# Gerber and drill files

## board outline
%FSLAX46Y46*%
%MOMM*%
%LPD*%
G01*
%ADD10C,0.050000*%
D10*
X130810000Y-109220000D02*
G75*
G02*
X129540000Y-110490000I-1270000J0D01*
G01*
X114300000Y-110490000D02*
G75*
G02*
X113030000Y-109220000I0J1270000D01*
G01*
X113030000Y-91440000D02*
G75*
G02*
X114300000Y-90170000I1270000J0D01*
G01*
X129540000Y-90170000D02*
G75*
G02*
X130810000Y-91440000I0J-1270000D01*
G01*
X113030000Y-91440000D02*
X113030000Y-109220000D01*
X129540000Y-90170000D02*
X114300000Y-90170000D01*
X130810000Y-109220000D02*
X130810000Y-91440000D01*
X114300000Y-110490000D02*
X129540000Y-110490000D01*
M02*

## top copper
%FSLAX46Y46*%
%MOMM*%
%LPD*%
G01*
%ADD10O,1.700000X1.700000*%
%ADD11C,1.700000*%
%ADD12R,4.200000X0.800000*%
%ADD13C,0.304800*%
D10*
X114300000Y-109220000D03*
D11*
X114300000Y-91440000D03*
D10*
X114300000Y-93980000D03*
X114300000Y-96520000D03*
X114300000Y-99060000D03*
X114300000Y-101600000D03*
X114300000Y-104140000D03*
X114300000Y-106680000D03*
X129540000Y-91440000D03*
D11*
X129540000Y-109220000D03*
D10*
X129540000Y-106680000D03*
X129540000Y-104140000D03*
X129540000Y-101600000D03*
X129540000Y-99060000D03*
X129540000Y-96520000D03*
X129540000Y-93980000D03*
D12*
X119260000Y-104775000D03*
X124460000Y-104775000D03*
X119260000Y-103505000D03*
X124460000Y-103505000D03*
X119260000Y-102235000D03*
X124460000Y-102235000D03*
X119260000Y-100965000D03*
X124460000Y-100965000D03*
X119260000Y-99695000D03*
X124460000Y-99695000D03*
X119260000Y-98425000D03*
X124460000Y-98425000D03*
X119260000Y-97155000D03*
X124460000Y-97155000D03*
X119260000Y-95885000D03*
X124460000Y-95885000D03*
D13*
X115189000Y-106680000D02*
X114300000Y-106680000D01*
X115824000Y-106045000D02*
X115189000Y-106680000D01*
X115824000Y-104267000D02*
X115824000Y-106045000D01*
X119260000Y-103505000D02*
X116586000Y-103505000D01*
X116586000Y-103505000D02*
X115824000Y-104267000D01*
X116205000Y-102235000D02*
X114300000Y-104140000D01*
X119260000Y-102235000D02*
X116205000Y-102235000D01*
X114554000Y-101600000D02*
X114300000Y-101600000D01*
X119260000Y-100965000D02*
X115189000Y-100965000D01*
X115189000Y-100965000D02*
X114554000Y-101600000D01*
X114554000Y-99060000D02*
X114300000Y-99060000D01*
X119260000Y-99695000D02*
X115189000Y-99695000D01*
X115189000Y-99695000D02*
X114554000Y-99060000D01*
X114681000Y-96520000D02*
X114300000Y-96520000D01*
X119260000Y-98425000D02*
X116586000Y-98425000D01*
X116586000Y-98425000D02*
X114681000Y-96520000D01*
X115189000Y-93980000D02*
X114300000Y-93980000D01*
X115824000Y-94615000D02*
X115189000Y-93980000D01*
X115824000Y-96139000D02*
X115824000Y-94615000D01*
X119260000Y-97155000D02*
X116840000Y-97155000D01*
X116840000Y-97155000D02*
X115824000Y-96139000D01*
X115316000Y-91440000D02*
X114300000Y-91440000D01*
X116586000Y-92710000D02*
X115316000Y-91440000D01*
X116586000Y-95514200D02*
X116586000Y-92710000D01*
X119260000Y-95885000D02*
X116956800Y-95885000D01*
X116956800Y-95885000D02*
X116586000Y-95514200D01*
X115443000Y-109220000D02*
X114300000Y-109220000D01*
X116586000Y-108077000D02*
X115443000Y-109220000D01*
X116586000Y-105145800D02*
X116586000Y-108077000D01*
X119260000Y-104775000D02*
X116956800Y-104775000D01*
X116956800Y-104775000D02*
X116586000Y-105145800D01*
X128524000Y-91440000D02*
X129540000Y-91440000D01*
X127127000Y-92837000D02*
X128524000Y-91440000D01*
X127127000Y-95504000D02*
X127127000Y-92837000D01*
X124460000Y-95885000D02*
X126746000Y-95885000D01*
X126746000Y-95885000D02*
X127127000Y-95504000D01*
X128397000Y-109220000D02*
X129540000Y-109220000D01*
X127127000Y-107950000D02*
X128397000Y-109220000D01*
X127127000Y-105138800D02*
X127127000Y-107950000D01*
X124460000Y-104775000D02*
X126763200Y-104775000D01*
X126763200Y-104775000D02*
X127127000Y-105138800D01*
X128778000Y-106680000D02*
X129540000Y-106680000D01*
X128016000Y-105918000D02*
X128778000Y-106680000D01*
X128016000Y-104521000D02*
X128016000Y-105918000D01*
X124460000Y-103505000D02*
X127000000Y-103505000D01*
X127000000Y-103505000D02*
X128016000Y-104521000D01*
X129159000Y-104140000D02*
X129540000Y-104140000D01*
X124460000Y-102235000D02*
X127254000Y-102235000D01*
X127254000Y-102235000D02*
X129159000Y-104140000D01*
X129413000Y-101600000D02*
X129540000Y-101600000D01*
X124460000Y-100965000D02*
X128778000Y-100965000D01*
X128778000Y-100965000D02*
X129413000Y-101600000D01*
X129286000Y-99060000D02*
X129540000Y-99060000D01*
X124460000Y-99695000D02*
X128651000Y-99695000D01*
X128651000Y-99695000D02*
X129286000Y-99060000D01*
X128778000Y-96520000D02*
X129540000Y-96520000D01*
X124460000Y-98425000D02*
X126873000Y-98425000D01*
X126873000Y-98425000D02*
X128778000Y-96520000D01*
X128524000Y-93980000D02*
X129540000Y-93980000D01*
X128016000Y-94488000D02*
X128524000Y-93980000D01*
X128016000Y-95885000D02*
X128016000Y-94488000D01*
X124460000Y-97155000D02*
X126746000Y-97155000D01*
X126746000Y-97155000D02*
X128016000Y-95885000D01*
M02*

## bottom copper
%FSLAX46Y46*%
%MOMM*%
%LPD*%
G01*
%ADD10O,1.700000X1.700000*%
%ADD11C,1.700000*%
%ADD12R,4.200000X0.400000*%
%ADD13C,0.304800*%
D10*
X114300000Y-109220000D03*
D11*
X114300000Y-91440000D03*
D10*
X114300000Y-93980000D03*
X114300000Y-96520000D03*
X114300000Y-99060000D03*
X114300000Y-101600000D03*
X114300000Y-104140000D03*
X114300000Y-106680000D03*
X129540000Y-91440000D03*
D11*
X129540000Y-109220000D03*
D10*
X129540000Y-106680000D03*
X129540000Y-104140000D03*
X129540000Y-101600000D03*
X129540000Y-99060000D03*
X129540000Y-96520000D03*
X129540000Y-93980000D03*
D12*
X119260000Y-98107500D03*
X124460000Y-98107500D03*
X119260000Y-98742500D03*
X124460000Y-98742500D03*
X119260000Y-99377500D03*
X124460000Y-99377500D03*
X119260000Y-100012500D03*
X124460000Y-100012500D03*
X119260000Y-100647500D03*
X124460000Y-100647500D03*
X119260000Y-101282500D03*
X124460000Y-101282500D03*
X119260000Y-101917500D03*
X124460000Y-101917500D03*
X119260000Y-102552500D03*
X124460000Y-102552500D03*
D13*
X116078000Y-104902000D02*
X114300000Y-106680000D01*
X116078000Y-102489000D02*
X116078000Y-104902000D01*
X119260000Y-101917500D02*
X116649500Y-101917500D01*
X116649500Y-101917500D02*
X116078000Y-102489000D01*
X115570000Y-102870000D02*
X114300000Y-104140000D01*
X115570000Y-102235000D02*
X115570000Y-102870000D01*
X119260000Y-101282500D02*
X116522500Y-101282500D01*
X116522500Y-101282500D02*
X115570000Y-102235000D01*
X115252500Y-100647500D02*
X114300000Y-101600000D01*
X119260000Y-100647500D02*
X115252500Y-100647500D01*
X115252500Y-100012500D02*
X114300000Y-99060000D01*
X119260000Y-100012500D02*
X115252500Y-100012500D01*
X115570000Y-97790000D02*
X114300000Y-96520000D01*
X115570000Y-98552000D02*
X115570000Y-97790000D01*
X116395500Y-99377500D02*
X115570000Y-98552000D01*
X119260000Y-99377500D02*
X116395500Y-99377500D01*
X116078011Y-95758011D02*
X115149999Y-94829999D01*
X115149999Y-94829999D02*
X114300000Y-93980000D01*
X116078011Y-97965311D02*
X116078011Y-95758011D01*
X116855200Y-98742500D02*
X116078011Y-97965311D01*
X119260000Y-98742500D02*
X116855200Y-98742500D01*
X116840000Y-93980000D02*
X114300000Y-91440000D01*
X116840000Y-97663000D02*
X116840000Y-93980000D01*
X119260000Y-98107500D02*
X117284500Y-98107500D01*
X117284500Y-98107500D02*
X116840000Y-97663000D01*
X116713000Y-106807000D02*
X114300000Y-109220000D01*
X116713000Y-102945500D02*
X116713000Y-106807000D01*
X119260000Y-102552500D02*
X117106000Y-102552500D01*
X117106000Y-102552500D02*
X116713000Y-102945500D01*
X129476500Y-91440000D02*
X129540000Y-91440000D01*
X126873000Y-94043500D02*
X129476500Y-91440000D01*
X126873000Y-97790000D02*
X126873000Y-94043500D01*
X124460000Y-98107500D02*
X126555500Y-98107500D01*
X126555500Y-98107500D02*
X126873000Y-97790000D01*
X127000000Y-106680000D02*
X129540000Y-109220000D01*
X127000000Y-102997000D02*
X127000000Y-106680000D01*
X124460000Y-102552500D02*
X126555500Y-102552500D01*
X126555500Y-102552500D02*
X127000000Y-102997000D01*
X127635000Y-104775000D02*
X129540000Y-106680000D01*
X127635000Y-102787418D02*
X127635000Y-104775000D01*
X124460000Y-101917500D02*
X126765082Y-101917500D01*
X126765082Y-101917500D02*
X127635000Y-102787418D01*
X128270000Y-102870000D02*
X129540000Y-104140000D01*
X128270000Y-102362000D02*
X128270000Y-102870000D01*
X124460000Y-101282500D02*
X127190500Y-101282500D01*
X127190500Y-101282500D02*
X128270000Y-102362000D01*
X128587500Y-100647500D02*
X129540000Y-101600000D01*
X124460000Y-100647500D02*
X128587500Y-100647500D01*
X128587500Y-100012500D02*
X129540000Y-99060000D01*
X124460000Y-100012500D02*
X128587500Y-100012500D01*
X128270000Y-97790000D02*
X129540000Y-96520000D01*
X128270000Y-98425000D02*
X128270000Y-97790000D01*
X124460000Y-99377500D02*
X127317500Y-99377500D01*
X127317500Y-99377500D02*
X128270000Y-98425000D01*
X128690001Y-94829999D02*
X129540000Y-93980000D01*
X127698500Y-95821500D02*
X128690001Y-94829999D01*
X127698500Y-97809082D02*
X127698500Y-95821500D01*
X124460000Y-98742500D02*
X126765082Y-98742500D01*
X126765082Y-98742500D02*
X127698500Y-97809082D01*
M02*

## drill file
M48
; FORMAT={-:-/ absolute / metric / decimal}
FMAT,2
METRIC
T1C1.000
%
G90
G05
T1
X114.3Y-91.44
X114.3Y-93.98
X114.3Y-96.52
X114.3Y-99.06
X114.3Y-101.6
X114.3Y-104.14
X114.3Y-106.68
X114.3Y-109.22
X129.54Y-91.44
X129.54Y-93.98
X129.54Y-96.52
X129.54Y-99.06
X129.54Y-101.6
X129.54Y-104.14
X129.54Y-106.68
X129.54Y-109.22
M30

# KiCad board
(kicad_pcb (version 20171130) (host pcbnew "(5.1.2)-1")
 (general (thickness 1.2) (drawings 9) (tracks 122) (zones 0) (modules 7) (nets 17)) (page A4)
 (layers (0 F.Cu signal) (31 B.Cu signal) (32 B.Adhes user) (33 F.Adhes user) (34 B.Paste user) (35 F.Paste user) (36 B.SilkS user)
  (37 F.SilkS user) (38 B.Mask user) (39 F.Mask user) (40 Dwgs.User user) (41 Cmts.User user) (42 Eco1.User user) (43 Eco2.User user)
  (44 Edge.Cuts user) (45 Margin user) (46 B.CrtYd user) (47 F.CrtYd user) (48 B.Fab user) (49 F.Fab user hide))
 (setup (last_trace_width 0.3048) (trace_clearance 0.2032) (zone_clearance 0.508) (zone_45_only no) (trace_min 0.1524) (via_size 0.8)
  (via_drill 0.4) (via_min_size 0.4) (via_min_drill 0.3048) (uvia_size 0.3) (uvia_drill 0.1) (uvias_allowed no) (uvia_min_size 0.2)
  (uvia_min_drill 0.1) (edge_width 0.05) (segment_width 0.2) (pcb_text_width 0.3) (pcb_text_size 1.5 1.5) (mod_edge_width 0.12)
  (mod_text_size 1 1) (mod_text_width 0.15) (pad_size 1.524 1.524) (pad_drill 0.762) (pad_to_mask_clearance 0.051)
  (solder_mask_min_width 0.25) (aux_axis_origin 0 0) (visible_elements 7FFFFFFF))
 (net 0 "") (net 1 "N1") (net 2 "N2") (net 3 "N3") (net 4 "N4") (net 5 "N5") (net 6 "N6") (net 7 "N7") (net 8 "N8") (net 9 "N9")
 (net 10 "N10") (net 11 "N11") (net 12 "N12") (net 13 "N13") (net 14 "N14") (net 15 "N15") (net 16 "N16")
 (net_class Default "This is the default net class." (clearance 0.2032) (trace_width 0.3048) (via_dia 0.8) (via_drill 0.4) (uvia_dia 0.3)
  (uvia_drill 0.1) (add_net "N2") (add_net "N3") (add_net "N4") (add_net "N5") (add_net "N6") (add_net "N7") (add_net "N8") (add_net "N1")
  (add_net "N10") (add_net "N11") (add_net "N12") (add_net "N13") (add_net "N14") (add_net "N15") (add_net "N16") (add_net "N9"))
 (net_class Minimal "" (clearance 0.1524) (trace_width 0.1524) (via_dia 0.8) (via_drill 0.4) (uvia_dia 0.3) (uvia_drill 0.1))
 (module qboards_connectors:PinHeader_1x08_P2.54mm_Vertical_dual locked (layer F.Cu) (at 114.3 91.44)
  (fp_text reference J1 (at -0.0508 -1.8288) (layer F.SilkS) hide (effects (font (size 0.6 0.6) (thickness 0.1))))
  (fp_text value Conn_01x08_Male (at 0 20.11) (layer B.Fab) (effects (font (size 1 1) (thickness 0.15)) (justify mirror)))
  (pad 8 thru_hole oval (at 0 17.78) (size 1.7 1.7) (drill 1) (layers *.Cu *.Mask) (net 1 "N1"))
  (pad 1 thru_hole circle (at 0 0) (size 1.7 1.7) (drill 1) (layers *.Cu *.Mask) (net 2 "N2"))
  (pad 2 thru_hole oval (at 0 2.54) (size 1.7 1.7) (drill 1) (layers *.Cu *.Mask) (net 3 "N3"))
  (pad 3 thru_hole oval (at 0 5.08) (size 1.7 1.7) (drill 1) (layers *.Cu *.Mask) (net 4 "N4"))
  (pad 4 thru_hole oval (at 0 7.62) (size 1.7 1.7) (drill 1) (layers *.Cu *.Mask) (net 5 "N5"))
  (pad 5 thru_hole oval (at 0 10.16) (size 1.7 1.7) (drill 1) (layers *.Cu *.Mask) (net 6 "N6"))
  (pad 6 thru_hole oval (at 0 12.7) (size 1.7 1.7) (drill 1) (layers *.Cu *.Mask) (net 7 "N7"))
  (pad 7 thru_hole oval (at 0 15.24) (size 1.7 1.7) (drill 1) (layers *.Cu *.Mask) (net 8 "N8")))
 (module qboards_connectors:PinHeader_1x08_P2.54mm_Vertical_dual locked (layer F.Cu) (at 129.54 109.22 180)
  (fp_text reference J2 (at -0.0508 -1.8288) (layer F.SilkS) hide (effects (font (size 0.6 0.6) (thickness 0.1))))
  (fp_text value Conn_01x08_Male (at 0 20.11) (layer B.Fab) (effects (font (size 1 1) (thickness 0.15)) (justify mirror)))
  (pad 8 thru_hole oval (at 0 17.78 180) (size 1.7 1.7) (drill 1) (layers *.Cu *.Mask) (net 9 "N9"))
  (pad 1 thru_hole circle (at 0 0 180) (size 1.7 1.7) (drill 1) (layers *.Cu *.Mask) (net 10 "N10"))
  (pad 2 thru_hole oval (at 0 2.54 180) (size 1.7 1.7) (drill 1) (layers *.Cu *.Mask) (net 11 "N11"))
  (pad 3 thru_hole oval (at 0 5.08 180) (size 1.7 1.7) (drill 1) (layers *.Cu *.Mask) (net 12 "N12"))
  (pad 4 thru_hole oval (at 0 7.62 180) (size 1.7 1.7) (drill 1) (layers *.Cu *.Mask) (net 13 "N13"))
  (pad 5 thru_hole oval (at 0 10.16 180) (size 1.7 1.7) (drill 1) (layers *.Cu *.Mask) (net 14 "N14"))
  (pad 6 thru_hole oval (at 0 12.7 180) (size 1.7 1.7) (drill 1) (layers *.Cu *.Mask) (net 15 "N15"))
  (pad 7 thru_hole oval (at 0 15.24 180) (size 1.7 1.7) (drill 1) (layers *.Cu *.Mask) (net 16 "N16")))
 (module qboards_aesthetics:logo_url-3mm (layer F.Cu) (at 117.602 107.823)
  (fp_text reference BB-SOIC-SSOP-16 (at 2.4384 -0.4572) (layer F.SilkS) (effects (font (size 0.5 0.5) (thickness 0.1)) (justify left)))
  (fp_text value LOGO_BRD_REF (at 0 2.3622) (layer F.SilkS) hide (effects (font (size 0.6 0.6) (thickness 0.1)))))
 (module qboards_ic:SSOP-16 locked (layer B.Cu) (at 121.86 100.33 90)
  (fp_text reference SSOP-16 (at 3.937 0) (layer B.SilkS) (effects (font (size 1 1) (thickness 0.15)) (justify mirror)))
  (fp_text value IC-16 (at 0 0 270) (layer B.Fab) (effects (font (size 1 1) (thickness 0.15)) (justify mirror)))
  (pad 8 smd rect (at 2.2225 -2.6 90) (size 0.4 4.2) (layers B.Cu B.Paste B.Mask) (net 2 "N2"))
  (pad 9 smd rect (at 2.2225 2.6 90) (size 0.4 4.2) (layers B.Cu B.Paste B.Mask) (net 9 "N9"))
  (pad 7 smd rect (at 1.5875 -2.6 90) (size 0.4 4.2) (layers B.Cu B.Paste B.Mask) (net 3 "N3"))
  (pad 10 smd rect (at 1.5875 2.6 90) (size 0.4 4.2) (layers B.Cu B.Paste B.Mask) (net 16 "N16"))
  (pad 6 smd rect (at 0.9525 -2.6 90) (size 0.4 4.2) (layers B.Cu B.Paste B.Mask) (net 4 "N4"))
  (pad 11 smd rect (at 0.9525 2.6 90) (size 0.4 4.2) (layers B.Cu B.Paste B.Mask) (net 15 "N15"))
  (pad 5 smd rect (at 0.3175 -2.6 90) (size 0.4 4.2) (layers B.Cu B.Paste B.Mask) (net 5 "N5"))
  (pad 12 smd rect (at 0.3175 2.6 90) (size 0.4 4.2) (layers B.Cu B.Paste B.Mask) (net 14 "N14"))
  (pad 4 smd rect (at -0.3175 -2.6 90) (size 0.4 4.2) (layers B.Cu B.Paste B.Mask) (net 6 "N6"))
  (pad 13 smd rect (at -0.3175 2.6 90) (size 0.4 4.2) (layers B.Cu B.Paste B.Mask) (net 13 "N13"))
  (pad 3 smd rect (at -0.9525 -2.6 90) (size 0.4 4.2) (layers B.Cu B.Paste B.Mask) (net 7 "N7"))
  (pad 14 smd rect (at -0.9525 2.6 90) (size 0.4 4.2) (layers B.Cu B.Paste B.Mask) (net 12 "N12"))
  (pad 2 smd rect (at -1.5875 -2.6 90) (size 0.4 4.2) (layers B.Cu B.Paste B.Mask) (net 8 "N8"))
  (pad 15 smd rect (at -1.5875 2.6 90) (size 0.4 4.2) (layers B.Cu B.Paste B.Mask) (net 11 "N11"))
  (pad 1 smd rect (at -2.2225 -2.6 90) (size 0.4 4.2) (layers B.Cu B.Paste B.Mask) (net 1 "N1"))
  (pad 16 smd rect (at -2.2225 2.6 90) (size 0.4 4.2) (layers B.Cu B.Paste B.Mask) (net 10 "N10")))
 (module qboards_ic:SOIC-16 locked (layer F.Cu) (at 121.86 100.33 270)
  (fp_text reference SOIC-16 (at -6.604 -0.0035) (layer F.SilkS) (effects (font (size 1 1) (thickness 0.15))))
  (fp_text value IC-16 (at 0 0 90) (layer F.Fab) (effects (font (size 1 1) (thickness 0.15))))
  (pad 8 smd rect (at 4.445 2.6 270) (size 0.8 4.2) (layers F.Cu F.Paste F.Mask) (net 1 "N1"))
  (pad 9 smd rect (at 4.445 -2.6 270) (size 0.8 4.2) (layers F.Cu F.Paste F.Mask) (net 10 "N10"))
  (pad 7 smd rect (at 3.175 2.6 270) (size 0.8 4.2) (layers F.Cu F.Paste F.Mask) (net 8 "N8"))
  (pad 10 smd rect (at 3.175 -2.6 270) (size 0.8 4.2) (layers F.Cu F.Paste F.Mask) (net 11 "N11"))
  (pad 6 smd rect (at 1.905 2.6 270) (size 0.8 4.2) (layers F.Cu F.Paste F.Mask) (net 7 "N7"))
  (pad 11 smd rect (at 1.905 -2.6 270) (size 0.8 4.2) (layers F.Cu F.Paste F.Mask) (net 12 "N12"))
  (pad 5 smd rect (at 0.635 2.6 270) (size 0.8 4.2) (layers F.Cu F.Paste F.Mask) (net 6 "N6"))
  (pad 12 smd rect (at 0.635 -2.6 270) (size 0.8 4.2) (layers F.Cu F.Paste F.Mask) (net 13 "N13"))
  (pad 4 smd rect (at -0.635 2.6 270) (size 0.8 4.2) (layers F.Cu F.Paste F.Mask) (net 5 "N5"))
  (pad 13 smd rect (at -0.635 -2.6 270) (size 0.8 4.2) (layers F.Cu F.Paste F.Mask) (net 14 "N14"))
  (pad 3 smd rect (at -1.905 2.6 270) (size 0.8 4.2) (layers F.Cu F.Paste F.Mask) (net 4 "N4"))
  (pad 14 smd rect (at -1.905 -2.6 270) (size 0.8 4.2) (layers F.Cu F.Paste F.Mask) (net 15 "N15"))
  (pad 2 smd rect (at -3.175 2.6 270) (size 0.8 4.2) (layers F.Cu F.Paste F.Mask) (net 3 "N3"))
  (pad 15 smd rect (at -3.175 -2.6 270) (size 0.8 4.2) (layers F.Cu F.Paste F.Mask) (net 16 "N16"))
  (pad 1 smd rect (at -4.445 2.6 270) (size 0.8 4.2) (layers F.Cu F.Paste F.Mask) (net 2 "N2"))
  (pad 16 smd rect (at -4.445 -2.6 270) (size 0.8 4.2) (layers F.Cu F.Paste F.Mask) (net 9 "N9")))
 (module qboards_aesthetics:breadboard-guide (layer F.Cu) (at 99.06 91.44)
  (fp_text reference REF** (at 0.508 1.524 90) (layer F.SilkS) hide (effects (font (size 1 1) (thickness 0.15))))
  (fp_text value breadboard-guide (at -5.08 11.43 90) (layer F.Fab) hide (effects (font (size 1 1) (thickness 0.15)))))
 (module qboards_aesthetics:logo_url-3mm (layer B.Cu) (at 126.492 107.823 180)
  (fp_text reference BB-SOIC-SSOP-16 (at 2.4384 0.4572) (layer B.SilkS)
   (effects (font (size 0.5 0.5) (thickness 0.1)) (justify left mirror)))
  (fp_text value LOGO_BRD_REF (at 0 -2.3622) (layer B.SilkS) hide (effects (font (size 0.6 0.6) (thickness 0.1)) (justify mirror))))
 (gr_arc (start 129.54 109.22) (end 129.54 110.49) (angle -90) (layer Edge.Cuts) (width 0.05))
 (gr_arc (start 114.3 109.22) (end 113.03 109.22) (angle -90) (layer Edge.Cuts) (width 0.05))
 (gr_arc (start 114.3 91.44) (end 114.3 90.17) (angle -90) (layer Edge.Cuts) (width 0.05))
 (gr_arc (start 129.54 91.44) (end 130.81 91.44) (angle -90) (layer Edge.Cuts) (width 0.05))
 (gr_line (start 113.03 91.44) (end 113.03 109.22) (layer Edge.Cuts) (width 0.05))
 (gr_line (start 129.54 90.17) (end 114.3 90.17) (layer Edge.Cuts) (width 0.05))
 (gr_line (start 130.81 109.22) (end 130.81 91.44) (layer Edge.Cuts) (width 0.05))
 (gr_line (start 114.3 110.49) (end 129.54 110.49) (layer Edge.Cuts) (width 0.05))
 (segment (start 115.189 106.68) (end 114.3 106.68) (width 0.3048) (layer F.Cu) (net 8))
 (segment (start 115.824 106.045) (end 115.189 106.68) (width 0.3048) (layer F.Cu) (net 8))
 (segment (start 115.824 104.267) (end 115.824 106.045) (width 0.3048) (layer F.Cu) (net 8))
 (segment (start 119.26 103.505) (end 116.586 103.505) (width 0.3048) (layer F.Cu) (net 8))
 (segment (start 116.586 103.505) (end 115.824 104.267) (width 0.3048) (layer F.Cu) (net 8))
 (segment (start 116.078 104.902) (end 114.3 106.68) (width 0.3048) (layer B.Cu) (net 8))
 (segment (start 116.078 102.489) (end 116.078 104.902) (width 0.3048) (layer B.Cu) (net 8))
 (segment (start 119.26 101.9175) (end 116.6495 101.9175) (width 0.3048) (layer B.Cu) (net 8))
 (segment (start 116.6495 101.9175) (end 116.078 102.489) (width 0.3048) (layer B.Cu) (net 8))
 (segment (start 116.205 102.235) (end 114.3 104.14) (width 0.3048) (layer F.Cu) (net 7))
 (segment (start 119.26 102.235) (end 116.205 102.235) (width 0.3048) (layer F.Cu) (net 7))
 (segment (start 115.57 102.87) (end 114.3 104.14) (width 0.3048) (layer B.Cu) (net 7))
 (segment (start 115.57 102.235) (end 115.57 102.87) (width 0.3048) (layer B.Cu) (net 7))
 (segment (start 119.26 101.2825) (end 116.5225 101.2825) (width 0.3048) (layer B.Cu) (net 7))
 (segment (start 116.5225 101.2825) (end 115.57 102.235) (width 0.3048) (layer B.Cu) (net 7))
 (segment (start 114.554 101.6) (end 114.3 101.6) (width 0.3048) (layer F.Cu) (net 6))
 (segment (start 119.26 100.965) (end 115.189 100.965) (width 0.3048) (layer F.Cu) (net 6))
 (segment (start 115.189 100.965) (end 114.554 101.6) (width 0.3048) (layer F.Cu) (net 6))
 (segment (start 115.2525 100.6475) (end 114.3 101.6) (width 0.3048) (layer B.Cu) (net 6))
 (segment (start 119.26 100.6475) (end 115.2525 100.6475) (width 0.3048) (layer B.Cu) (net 6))
 (segment (start 114.554 99.06) (end 114.3 99.06) (width 0.3048) (layer F.Cu) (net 5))
 (segment (start 119.26 99.695) (end 115.189 99.695) (width 0.3048) (layer F.Cu) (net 5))
 (segment (start 115.189 99.695) (end 114.554 99.06) (width 0.3048) (layer F.Cu) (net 5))
 (segment (start 115.2525 100.0125) (end 114.3 99.06) (width 0.3048) (layer B.Cu) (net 5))
 (segment (start 119.26 100.0125) (end 115.2525 100.0125) (width 0.3048) (layer B.Cu) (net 5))
 (segment (start 114.681 96.52) (end 114.3 96.52) (width 0.3048) (layer F.Cu) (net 4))
 (segment (start 119.26 98.425) (end 116.586 98.425) (width 0.3048) (layer F.Cu) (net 4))
 (segment (start 116.586 98.425) (end 114.681 96.52) (width 0.3048) (layer F.Cu) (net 4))
 (segment (start 115.57 97.79) (end 114.3 96.52) (width 0.3048) (layer B.Cu) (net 4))
 (segment (start 115.57 98.552) (end 115.57 97.79) (width 0.3048) (layer B.Cu) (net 4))
 (segment (start 116.3955 99.3775) (end 115.57 98.552) (width 0.3048) (layer B.Cu) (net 4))
 (segment (start 119.26 99.3775) (end 116.3955 99.3775) (width 0.3048) (layer B.Cu) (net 4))
 (segment (start 115.189 93.98) (end 114.3 93.98) (width 0.3048) (layer F.Cu) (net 3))
 (segment (start 115.824 94.615) (end 115.189 93.98) (width 0.3048) (layer F.Cu) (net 3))
 (segment (start 115.824 96.139) (end 115.824 94.615) (width 0.3048) (layer F.Cu) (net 3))
 (segment (start 119.26 97.155) (end 116.84 97.155) (width 0.3048) (layer F.Cu) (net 3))
 (segment (start 116.84 97.155) (end 115.824 96.139) (width 0.3048) (layer F.Cu) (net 3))
 (segment (start 116.078011 95.758011) (end 115.149999 94.829999) (width 0.3048) (layer B.Cu) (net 3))
 (segment (start 115.149999 94.829999) (end 114.3 93.98) (width 0.3048) (layer B.Cu) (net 3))
 (segment (start 116.078011 97.965311) (end 116.078011 95.758011) (width 0.3048) (layer B.Cu) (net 3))
 (segment (start 116.8552 98.7425) (end 116.078011 97.965311) (width 0.3048) (layer B.Cu) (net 3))
 (segment (start 119.26 98.7425) (end 116.8552 98.7425) (width 0.3048) (layer B.Cu) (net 3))
 (segment (start 115.316 91.44) (end 114.3 91.44) (width 0.3048) (layer F.Cu) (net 2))
 (segment (start 116.586 92.71) (end 115.316 91.44) (width 0.3048) (layer F.Cu) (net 2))
 (segment (start 116.586 95.5142) (end 116.586 92.71) (width 0.3048) (layer F.Cu) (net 2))
 (segment (start 119.26 95.885) (end 116.9568 95.885) (width 0.3048) (layer F.Cu) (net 2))
 (segment (start 116.9568 95.885) (end 116.586 95.5142) (width 0.3048) (layer F.Cu) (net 2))
 (segment (start 116.84 93.98) (end 114.3 91.44) (width 0.3048) (layer B.Cu) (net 2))
 (segment (start 116.84 97.663) (end 116.84 93.98) (width 0.3048) (layer B.Cu) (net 2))
 (segment (start 119.26 98.1075) (end 117.2845 98.1075) (width 0.3048) (layer B.Cu) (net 2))
 (segment (start 117.2845 98.1075) (end 116.84 97.663) (width 0.3048) (layer B.Cu) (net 2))
 (segment (start 115.443 109.22) (end 114.3 109.22) (width 0.3048) (layer F.Cu) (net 1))
 (segment (start 116.586 108.077) (end 115.443 109.22) (width 0.3048) (layer F.Cu) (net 1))
 (segment (start 116.586 105.1458) (end 116.586 108.077) (width 0.3048) (layer F.Cu) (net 1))
 (segment (start 119.26 104.775) (end 116.9568 104.775) (width 0.3048) (layer F.Cu) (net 1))
 (segment (start 116.9568 104.775) (end 116.586 105.1458) (width 0.3048) (layer F.Cu) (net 1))
 (segment (start 116.713 106.807) (end 114.3 109.22) (width 0.3048) (layer B.Cu) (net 1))
 (segment (start 116.713 102.9455) (end 116.713 106.807) (width 0.3048) (layer B.Cu) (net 1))
 (segment (start 119.26 102.5525) (end 117.106 102.5525) (width 0.3048) (layer B.Cu) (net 1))
 (segment (start 117.106 102.5525) (end 116.713 102.9455) (width 0.3048) (layer B.Cu) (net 1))
 (segment (start 128.524 91.44) (end 129.54 91.44) (width 0.3048) (layer F.Cu) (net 9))
 (segment (start 127.127 92.837) (end 128.524 91.44) (width 0.3048) (layer F.Cu) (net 9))
 (segment (start 127.127 95.504) (end 127.127 92.837) (width 0.3048) (layer F.Cu) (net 9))
 (segment (start 124.46 95.885) (end 126.746 95.885) (width 0.3048) (layer F.Cu) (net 9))
 (segment (start 126.746 95.885) (end 127.127 95.504) (width 0.3048) (layer F.Cu) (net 9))
 (segment (start 129.4765 91.44) (end 129.54 91.44) (width 0.3048) (layer B.Cu) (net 9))
 (segment (start 126.873 94.0435) (end 129.4765 91.44) (width 0.3048) (layer B.Cu) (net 9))
 (segment (start 126.873 97.79) (end 126.873 94.0435) (width 0.3048) (layer B.Cu) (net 9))
 (segment (start 124.46 98.1075) (end 126.5555 98.1075) (width 0.3048) (layer B.Cu) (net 9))
 (segment (start 126.5555 98.1075) (end 126.873 97.79) (width 0.3048) (layer B.Cu) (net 9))
 (segment (start 128.397 109.22) (end 129.54 109.22) (width 0.3048) (layer F.Cu) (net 10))
 (segment (start 127.127 107.95) (end 128.397 109.22) (width 0.3048) (layer F.Cu) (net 10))
 (segment (start 127.127 105.1388) (end 127.127 107.95) (width 0.3048) (layer F.Cu) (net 10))
 (segment (start 124.46 104.775) (end 126.7632 104.775) (width 0.3048) (layer F.Cu) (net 10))
 (segment (start 126.7632 104.775) (end 127.127 105.1388) (width 0.3048) (layer F.Cu) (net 10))
 (segment (start 127 106.68) (end 129.54 109.22) (width 0.3048) (layer B.Cu) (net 10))
 (segment (start 127 102.997) (end 127 106.68) (width 0.3048) (layer B.Cu) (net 10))
 (segment (start 124.46 102.5525) (end 126.5555 102.5525) (width 0.3048) (layer B.Cu) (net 10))
 (segment (start 126.5555 102.5525) (end 127 102.997) (width 0.3048) (layer B.Cu) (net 10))
 (segment (start 128.778 106.68) (end 129.54 106.68) (width 0.3048) (layer F.Cu) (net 11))
 (segment (start 128.016 105.918) (end 128.778 106.68) (width 0.3048) (layer F.Cu) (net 11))
 (segment (start 128.016 104.521) (end 128.016 105.918) (width 0.3048) (layer F.Cu) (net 11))
 (segment (start 124.46 103.505) (end 127 103.505) (width 0.3048) (layer F.Cu) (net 11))
 (segment (start 127 103.505) (end 128.016 104.521) (width 0.3048) (layer F.Cu) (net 11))
 (segment (start 127.635 104.775) (end 129.54 106.68) (width 0.3048) (layer B.Cu) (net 11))
 (segment (start 127.635 102.787418) (end 127.635 104.775) (width 0.3048) (layer B.Cu) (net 11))
 (segment (start 124.46 101.9175) (end 126.765082 101.9175) (width 0.3048) (layer B.Cu) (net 11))
 (segment (start 126.765082 101.9175) (end 127.635 102.787418) (width 0.3048) (layer B.Cu) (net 11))
 (segment (start 129.159 104.14) (end 129.54 104.14) (width 0.3048) (layer F.Cu) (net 12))
 (segment (start 124.46 102.235) (end 127.254 102.235) (width 0.3048) (layer F.Cu) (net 12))
 (segment (start 127.254 102.235) (end 129.159 104.14) (width 0.3048) (layer F.Cu) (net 12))
 (segment (start 128.27 102.87) (end 129.54 104.14) (width 0.3048) (layer B.Cu) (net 12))
 (segment (start 128.27 102.362) (end 128.27 102.87) (width 0.3048) (layer B.Cu) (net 12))
 (segment (start 124.46 101.2825) (end 127.1905 101.2825) (width 0.3048) (layer B.Cu) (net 12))
 (segment (start 127.1905 101.2825) (end 128.27 102.362) (width 0.3048) (layer B.Cu) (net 12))
 (segment (start 129.413 101.6) (end 129.54 101.6) (width 0.3048) (layer F.Cu) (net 13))
 (segment (start 124.46 100.965) (end 128.778 100.965) (width 0.3048) (layer F.Cu) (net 13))
 (segment (start 128.778 100.965) (end 129.413 101.6) (width 0.3048) (layer F.Cu) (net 13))
 (segment (start 128.5875 100.6475) (end 129.54 101.6) (width 0.3048) (layer B.Cu) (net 13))
 (segment (start 124.46 100.6475) (end 128.5875 100.6475) (width 0.3048) (layer B.Cu) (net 13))
 (segment (start 129.286 99.06) (end 129.54 99.06) (width 0.3048) (layer F.Cu) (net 14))
 (segment (start 124.46 99.695) (end 128.651 99.695) (width 0.3048) (layer F.Cu) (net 14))
 (segment (start 128.651 99.695) (end 129.286 99.06) (width 0.3048) (layer F.Cu) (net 14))
 (segment (start 128.5875 100.0125) (end 129.54 99.06) (width 0.3048) (layer B.Cu) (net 14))
 (segment (start 124.46 100.0125) (end 128.5875 100.0125) (width 0.3048) (layer B.Cu) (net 14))
 (segment (start 128.778 96.52) (end 129.54 96.52) (width 0.3048) (layer F.Cu) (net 15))
 (segment (start 124.46 98.425) (end 126.873 98.425) (width 0.3048) (layer F.Cu) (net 15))
 (segment (start 126.873 98.425) (end 128.778 96.52) (width 0.3048) (layer F.Cu) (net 15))
 (segment (start 128.27 97.79) (end 129.54 96.52) (width 0.3048) (layer B.Cu) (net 15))
 (segment (start 128.27 98.425) (end 128.27 97.79) (width 0.3048) (layer B.Cu) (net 15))
 (segment (start 124.46 99.3775) (end 127.3175 99.3775) (width 0.3048) (layer B.Cu) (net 15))
 (segment (start 127.3175 99.3775) (end 128.27 98.425) (width 0.3048) (layer B.Cu) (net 15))
 (segment (start 128.524 93.98) (end 129.54 93.98) (width 0.3048) (layer F.Cu) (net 16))
 (segment (start 128.016 94.488) (end 128.524 93.98) (width 0.3048) (layer F.Cu) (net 16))
 (segment (start 128.016 95.885) (end 128.016 94.488) (width 0.3048) (layer F.Cu) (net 16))
 (segment (start 124.46 97.155) (end 126.746 97.155) (width 0.3048) (layer F.Cu) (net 16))
 (segment (start 126.746 97.155) (end 128.016 95.885) (width 0.3048) (layer F.Cu) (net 16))
 (segment (start 128.690001 94.829999) (end 129.54 93.98) (width 0.3048) (layer B.Cu) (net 16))
 (segment (start 127.6985 95.8215) (end 128.690001 94.829999) (width 0.3048) (layer B.Cu) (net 16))
 (segment (start 127.6985 97.809082) (end 127.6985 95.8215) (width 0.3048) (layer B.Cu) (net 16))
 (segment (start 124.46 98.7425) (end 126.765082 98.7425) (width 0.3048) (layer B.Cu) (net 16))
 (segment (start 126.765082 98.7425) (end 127.6985 97.809082) (width 0.3048) (layer B.Cu) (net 16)))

